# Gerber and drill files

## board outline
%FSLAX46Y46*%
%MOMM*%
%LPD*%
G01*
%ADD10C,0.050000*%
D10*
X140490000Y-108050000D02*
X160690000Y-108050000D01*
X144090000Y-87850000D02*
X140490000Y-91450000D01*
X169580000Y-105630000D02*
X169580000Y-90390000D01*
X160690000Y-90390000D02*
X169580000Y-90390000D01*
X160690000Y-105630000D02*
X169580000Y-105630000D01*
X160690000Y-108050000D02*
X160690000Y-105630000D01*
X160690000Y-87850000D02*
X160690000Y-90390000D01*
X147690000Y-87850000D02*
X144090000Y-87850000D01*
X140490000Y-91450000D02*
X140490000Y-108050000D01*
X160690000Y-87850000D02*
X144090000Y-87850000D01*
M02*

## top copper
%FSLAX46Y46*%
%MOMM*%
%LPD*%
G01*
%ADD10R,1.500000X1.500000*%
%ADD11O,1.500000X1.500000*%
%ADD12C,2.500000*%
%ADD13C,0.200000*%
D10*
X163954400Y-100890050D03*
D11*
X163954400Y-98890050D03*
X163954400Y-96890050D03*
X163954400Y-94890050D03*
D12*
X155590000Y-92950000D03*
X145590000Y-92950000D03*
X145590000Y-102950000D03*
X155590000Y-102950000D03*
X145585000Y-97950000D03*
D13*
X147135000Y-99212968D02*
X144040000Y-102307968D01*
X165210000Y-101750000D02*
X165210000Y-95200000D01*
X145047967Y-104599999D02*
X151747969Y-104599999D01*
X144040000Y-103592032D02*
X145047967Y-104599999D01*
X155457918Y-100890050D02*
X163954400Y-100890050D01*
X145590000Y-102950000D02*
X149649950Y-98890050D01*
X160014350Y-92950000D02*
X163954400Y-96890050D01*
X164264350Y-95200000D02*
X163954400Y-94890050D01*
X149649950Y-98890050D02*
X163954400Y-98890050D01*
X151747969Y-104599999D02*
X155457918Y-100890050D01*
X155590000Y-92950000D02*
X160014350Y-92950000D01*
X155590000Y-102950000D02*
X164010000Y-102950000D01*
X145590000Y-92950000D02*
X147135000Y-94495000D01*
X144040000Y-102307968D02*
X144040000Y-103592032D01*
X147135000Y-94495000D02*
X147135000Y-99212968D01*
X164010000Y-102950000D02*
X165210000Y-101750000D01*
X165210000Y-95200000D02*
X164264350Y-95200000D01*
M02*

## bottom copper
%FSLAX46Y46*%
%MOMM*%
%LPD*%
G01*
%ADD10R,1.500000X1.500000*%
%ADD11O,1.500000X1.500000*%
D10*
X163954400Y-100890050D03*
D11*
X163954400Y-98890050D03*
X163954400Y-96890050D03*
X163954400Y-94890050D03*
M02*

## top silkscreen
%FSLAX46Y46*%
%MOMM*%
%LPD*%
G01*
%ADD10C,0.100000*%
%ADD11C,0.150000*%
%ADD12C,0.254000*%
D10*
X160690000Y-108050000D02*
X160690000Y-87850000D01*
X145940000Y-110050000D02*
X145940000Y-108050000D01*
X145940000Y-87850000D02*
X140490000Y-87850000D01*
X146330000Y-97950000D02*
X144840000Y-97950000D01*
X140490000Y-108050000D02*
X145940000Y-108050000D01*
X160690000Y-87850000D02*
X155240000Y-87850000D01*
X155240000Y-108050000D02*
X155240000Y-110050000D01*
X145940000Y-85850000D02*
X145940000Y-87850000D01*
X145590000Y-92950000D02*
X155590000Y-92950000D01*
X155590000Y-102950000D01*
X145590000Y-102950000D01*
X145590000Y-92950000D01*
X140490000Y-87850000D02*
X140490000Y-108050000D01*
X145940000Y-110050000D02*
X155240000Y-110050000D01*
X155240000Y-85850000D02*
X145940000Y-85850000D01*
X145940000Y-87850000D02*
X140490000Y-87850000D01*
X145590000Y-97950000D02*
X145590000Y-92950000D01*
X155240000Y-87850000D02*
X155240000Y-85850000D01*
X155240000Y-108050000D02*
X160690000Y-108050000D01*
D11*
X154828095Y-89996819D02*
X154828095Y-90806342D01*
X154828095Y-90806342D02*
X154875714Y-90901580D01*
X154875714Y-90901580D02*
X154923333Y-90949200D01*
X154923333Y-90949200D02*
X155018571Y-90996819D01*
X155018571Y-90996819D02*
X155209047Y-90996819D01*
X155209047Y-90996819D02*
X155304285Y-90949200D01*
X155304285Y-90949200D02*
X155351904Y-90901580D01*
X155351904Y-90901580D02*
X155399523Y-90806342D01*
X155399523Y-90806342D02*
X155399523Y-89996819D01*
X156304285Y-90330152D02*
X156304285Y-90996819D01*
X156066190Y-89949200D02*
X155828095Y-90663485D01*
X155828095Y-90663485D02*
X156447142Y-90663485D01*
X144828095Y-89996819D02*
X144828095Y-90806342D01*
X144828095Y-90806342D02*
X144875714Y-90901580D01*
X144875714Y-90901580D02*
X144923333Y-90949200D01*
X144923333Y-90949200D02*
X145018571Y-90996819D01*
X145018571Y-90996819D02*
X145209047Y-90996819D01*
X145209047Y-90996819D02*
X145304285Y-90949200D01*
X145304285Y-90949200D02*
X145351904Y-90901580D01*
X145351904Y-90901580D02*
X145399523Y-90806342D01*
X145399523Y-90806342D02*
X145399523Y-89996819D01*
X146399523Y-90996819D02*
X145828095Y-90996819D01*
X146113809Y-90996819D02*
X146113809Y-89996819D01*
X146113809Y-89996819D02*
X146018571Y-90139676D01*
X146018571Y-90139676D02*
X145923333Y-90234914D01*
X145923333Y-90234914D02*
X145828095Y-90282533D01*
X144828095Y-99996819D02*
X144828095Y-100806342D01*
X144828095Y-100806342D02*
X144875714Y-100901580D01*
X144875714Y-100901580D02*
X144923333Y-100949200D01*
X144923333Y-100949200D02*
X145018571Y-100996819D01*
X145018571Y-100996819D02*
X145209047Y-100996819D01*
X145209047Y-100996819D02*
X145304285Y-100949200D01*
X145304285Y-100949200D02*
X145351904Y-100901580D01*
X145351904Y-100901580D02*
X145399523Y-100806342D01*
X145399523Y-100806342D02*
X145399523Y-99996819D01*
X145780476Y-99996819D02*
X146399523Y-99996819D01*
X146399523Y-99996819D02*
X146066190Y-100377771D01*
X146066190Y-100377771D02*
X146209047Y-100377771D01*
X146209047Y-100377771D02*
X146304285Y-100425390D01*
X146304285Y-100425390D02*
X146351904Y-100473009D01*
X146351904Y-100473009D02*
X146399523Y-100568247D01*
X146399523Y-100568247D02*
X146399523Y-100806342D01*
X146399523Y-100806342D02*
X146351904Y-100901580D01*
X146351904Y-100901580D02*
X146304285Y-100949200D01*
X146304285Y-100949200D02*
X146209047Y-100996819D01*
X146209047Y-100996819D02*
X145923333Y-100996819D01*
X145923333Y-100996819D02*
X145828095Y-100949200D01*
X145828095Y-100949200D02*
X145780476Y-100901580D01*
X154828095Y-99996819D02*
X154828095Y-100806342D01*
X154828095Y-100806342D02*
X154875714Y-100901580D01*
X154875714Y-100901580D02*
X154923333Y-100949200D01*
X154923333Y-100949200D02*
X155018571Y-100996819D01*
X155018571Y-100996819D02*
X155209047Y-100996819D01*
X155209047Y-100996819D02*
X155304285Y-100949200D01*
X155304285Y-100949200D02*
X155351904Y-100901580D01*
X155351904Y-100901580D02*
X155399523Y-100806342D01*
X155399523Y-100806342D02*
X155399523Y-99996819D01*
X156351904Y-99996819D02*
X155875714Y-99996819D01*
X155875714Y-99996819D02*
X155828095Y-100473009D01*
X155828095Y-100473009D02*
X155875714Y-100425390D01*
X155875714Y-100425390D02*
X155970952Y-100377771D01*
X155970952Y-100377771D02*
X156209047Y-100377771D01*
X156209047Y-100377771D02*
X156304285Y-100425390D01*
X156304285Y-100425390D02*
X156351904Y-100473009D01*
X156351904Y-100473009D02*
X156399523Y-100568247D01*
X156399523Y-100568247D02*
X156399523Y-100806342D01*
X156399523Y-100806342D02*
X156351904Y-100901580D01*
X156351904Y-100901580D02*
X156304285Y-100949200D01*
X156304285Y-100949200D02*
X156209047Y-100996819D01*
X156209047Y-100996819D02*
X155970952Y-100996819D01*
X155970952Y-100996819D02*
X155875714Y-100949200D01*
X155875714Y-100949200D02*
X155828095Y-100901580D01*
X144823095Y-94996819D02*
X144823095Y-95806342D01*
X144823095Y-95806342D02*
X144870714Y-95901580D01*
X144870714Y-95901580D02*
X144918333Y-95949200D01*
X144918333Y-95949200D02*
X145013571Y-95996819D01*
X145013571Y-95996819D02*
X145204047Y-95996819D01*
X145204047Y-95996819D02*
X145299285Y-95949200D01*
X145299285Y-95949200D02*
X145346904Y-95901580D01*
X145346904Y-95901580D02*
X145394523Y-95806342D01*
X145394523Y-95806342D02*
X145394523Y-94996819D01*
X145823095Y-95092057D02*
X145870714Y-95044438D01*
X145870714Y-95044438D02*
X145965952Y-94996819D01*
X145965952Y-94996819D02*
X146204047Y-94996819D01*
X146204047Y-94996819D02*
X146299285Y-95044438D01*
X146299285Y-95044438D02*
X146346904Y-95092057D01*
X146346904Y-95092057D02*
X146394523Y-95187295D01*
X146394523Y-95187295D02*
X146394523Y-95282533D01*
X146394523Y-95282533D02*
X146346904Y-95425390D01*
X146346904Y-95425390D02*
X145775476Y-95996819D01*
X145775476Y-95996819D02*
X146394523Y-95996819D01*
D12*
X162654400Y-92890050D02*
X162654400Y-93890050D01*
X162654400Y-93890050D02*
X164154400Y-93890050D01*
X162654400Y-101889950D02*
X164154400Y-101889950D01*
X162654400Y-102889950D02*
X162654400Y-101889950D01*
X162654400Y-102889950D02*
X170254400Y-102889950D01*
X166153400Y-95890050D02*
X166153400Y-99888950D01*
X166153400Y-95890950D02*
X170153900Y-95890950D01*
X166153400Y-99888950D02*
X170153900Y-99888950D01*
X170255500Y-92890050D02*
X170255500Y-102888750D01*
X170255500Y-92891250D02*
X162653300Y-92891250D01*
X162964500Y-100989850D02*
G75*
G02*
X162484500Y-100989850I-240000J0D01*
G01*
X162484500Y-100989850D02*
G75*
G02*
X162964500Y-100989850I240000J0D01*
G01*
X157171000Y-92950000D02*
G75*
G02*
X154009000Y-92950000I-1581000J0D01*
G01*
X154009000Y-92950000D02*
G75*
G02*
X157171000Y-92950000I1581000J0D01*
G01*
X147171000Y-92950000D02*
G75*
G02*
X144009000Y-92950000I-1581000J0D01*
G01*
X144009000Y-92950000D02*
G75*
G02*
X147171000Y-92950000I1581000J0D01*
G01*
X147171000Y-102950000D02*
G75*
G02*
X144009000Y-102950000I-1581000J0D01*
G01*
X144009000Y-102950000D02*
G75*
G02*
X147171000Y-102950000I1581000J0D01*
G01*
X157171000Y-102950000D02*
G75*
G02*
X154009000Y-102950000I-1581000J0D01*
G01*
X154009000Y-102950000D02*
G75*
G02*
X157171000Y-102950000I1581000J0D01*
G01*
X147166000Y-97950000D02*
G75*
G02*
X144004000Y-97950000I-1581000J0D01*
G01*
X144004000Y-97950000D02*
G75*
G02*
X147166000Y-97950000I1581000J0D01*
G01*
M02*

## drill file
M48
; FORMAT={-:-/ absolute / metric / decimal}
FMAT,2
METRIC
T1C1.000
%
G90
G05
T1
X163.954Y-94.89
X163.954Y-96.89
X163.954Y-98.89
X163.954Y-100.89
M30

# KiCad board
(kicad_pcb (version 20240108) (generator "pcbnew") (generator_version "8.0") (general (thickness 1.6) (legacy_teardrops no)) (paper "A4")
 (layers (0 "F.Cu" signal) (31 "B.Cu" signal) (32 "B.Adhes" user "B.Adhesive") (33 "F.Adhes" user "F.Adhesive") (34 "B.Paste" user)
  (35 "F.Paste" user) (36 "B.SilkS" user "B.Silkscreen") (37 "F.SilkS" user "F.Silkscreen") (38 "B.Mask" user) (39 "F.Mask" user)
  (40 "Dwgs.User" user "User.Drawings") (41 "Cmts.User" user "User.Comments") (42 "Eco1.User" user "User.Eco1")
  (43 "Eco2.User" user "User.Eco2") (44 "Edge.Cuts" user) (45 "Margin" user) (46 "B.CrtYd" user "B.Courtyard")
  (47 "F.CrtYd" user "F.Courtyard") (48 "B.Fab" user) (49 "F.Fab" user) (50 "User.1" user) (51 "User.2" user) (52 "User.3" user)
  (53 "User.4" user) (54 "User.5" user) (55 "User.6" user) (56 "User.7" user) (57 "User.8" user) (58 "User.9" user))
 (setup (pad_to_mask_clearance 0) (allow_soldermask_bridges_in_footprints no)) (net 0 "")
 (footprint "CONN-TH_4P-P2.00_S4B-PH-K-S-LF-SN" (layer "F.Cu") (at 163.9544 97.89005 90)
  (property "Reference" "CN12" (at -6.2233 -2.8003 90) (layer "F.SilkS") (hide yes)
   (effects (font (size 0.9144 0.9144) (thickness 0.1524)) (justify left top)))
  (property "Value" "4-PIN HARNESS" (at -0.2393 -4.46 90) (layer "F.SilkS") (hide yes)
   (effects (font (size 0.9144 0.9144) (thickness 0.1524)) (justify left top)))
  (fp_line (start 5 -1.3) (end 4 -1.3) (stroke (width 0.254) (type default)) (layer "F.SilkS"))
  (fp_line (start 4 -1.3) (end 4 0.2) (stroke (width 0.254) (type default)) (layer "F.SilkS"))
  (fp_line (start -3.9999 -1.3) (end -3.9999 0.2) (stroke (width 0.254) (type default)) (layer "F.SilkS"))
  (fp_line (start -4.9999 -1.3) (end -3.9999 -1.3) (stroke (width 0.254) (type default)) (layer "F.SilkS"))
  (fp_line (start -4.9999 -1.3) (end -4.9999 6.3) (stroke (width 0.254) (type default)) (layer "F.SilkS"))
  (fp_line (start 2 2.199) (end -1.9989 2.199) (stroke (width 0.254) (type default)) (layer "F.SilkS"))
  (fp_line (start 1.9991 2.199) (end 1.9991 6.1995) (stroke (width 0.254) (type default)) (layer "F.SilkS"))
  (fp_line (start -1.9989 2.199) (end -1.9989 6.1995) (stroke (width 0.254) (type default)) (layer "F.SilkS"))
  (fp_line (start 5 6.3011) (end -4.9987 6.3011) (stroke (width 0.254) (type default)) (layer "F.SilkS"))
  (fp_line (start 4.9988 6.3011) (end 4.9988 -1.3011) (stroke (width 0.254) (type default)) (layer "F.SilkS"))
  (fp_circle (center -3.0998 -1.2299) (end -2.8598 -1.2299) (stroke (width 0.254) (type default)) (fill none) (layer "F.SilkS"))
  (pad "1" thru_hole rect (at -3 0 90) (size 1.5 1.5) (drill 1) (layers "*.Cu" "*.Mask") (remove_unused_layers no)
   (solder_mask_margin 0.0508) (thermal_bridge_angle 0))
  (pad "2" thru_hole oval (at -1 0 90) (size 1.5 1.5) (drill 1) (layers "*.Cu" "*.Mask") (remove_unused_layers no)
   (solder_mask_margin 0.0508) (thermal_bridge_angle 0))
  (pad "3" thru_hole oval (at 1 0 90) (size 1.5 1.5) (drill 1) (layers "*.Cu" "*.Mask") (remove_unused_layers no)
   (solder_mask_margin 0.0508) (thermal_bridge_angle 0))
  (pad "4" thru_hole oval (at 3 0 90) (size 1.5 1.5) (drill 1) (layers "*.Cu" "*.Mask") (remove_unused_layers no)
   (solder_mask_margin 0.0508) (thermal_bridge_angle 0))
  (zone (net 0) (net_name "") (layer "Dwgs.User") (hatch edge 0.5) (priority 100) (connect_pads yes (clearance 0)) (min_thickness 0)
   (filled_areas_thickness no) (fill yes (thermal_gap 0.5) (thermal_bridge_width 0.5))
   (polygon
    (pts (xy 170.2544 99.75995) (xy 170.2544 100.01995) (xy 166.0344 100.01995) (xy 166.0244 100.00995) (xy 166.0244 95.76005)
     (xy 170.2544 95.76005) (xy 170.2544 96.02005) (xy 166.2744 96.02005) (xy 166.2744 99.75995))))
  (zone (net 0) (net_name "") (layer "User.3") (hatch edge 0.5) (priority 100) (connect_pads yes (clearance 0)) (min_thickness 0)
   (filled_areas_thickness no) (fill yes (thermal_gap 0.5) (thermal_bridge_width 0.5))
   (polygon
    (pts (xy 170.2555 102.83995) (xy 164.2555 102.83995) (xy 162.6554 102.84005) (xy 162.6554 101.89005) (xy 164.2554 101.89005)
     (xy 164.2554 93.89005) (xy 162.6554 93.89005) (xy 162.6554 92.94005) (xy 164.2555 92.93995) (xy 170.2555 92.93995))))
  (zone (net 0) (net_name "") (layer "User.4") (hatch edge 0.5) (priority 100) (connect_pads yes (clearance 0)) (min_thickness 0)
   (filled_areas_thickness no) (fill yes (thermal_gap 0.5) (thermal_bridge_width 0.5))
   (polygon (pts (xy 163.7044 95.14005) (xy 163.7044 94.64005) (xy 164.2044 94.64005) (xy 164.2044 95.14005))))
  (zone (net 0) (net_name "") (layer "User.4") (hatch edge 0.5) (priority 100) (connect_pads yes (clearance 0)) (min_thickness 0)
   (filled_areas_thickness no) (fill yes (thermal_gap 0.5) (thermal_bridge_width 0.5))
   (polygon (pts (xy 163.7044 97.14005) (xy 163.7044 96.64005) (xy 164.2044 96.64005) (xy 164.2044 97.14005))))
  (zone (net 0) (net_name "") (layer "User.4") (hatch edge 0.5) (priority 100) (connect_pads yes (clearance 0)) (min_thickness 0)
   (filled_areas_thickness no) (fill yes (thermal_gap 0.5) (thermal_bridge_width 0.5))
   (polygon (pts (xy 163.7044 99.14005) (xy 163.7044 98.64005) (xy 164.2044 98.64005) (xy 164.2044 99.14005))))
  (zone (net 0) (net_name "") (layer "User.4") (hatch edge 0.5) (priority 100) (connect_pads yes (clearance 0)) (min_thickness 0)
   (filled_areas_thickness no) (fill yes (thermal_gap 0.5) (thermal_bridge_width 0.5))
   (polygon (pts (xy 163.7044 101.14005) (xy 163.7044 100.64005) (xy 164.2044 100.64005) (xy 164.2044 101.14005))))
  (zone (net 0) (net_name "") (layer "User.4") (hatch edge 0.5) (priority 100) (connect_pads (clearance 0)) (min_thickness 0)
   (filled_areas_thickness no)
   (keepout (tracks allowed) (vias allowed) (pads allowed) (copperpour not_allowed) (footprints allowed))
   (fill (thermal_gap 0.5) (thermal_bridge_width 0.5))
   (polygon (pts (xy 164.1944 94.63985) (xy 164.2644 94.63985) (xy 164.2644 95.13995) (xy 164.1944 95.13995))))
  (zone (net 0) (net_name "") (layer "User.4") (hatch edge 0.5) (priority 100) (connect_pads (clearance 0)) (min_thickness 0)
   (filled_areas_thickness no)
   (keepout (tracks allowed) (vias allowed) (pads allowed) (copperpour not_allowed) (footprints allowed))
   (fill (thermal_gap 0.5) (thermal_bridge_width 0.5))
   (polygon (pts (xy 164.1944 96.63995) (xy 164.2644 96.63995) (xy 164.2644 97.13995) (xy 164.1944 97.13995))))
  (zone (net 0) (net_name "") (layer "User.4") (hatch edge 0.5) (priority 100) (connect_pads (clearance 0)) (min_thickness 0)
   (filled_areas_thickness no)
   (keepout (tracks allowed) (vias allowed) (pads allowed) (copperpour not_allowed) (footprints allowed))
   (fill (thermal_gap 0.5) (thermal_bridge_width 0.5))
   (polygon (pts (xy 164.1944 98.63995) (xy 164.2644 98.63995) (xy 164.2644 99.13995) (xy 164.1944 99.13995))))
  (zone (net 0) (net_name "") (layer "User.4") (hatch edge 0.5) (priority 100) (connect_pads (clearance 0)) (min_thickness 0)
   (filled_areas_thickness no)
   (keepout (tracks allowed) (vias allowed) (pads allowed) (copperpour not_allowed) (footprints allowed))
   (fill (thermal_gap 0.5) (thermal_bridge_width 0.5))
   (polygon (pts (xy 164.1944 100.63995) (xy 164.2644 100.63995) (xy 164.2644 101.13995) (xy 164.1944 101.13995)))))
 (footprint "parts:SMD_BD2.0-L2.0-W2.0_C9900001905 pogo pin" (layer "F.Cu") (at 155.59 92.95)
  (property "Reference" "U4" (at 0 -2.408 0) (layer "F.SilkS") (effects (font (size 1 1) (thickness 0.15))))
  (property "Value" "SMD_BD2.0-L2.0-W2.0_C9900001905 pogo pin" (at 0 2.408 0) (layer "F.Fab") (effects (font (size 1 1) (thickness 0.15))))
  (fp_circle (center 0 0) (end 1.581 0) (stroke (width 0.254) (type default)) (fill none) (layer "F.SilkS"))
  (pad "1" smd circle (at 0 0) (size 2.5 2.5) (layers "F.Cu" "F.Paste" "F.Mask") (thermal_bridge_angle 90)))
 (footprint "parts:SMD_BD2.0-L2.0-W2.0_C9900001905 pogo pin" (layer "F.Cu") (at 145.59 92.95)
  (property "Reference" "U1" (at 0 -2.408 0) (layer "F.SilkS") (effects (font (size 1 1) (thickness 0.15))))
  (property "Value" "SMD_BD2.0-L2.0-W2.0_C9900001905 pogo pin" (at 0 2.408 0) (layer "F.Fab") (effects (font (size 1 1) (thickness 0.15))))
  (fp_circle (center 0 0) (end 1.581 0) (stroke (width 0.254) (type default)) (fill none) (layer "F.SilkS"))
  (pad "1" smd circle (at 0 0) (size 2.5 2.5) (layers "F.Cu" "F.Paste" "F.Mask") (thermal_bridge_angle 90)))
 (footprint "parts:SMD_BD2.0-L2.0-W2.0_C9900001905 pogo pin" (layer "F.Cu") (at 145.59 102.95)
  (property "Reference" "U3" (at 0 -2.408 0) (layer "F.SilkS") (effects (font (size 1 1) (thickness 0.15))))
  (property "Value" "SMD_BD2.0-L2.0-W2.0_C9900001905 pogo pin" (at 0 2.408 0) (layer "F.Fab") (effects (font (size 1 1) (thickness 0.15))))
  (fp_circle (center 0 0) (end 1.581 0) (stroke (width 0.254) (type default)) (fill none) (layer "F.SilkS"))
  (pad "1" smd circle (at 0 0) (size 2.5 2.5) (layers "F.Cu" "F.Paste" "F.Mask") (thermal_bridge_angle 90)))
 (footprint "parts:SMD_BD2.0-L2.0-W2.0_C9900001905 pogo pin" (layer "F.Cu") (at 155.59 102.95)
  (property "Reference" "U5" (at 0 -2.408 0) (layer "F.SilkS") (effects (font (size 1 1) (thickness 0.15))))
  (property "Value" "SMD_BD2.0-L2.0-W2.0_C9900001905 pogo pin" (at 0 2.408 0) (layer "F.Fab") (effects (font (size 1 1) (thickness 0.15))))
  (fp_circle (center 0 0) (end 1.581 0) (stroke (width 0.254) (type default)) (fill none) (layer "F.SilkS"))
  (pad "1" smd circle (at 0 0) (size 2.5 2.5) (layers "F.Cu" "F.Paste" "F.Mask") (thermal_bridge_angle 90)))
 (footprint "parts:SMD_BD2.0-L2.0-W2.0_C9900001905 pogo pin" (layer "F.Cu") (at 145.585 97.95)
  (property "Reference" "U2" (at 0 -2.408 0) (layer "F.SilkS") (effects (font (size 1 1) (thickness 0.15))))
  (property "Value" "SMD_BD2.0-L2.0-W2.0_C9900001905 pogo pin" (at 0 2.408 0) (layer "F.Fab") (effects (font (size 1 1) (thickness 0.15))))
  (fp_circle (center 0 0) (end 1.581 0) (stroke (width 0.254) (type default)) (fill none) (layer "F.SilkS"))
  (pad "1" smd circle (at 0 0) (size 2.5 2.5) (layers "F.Cu" "F.Paste" "F.Mask") (thermal_bridge_angle 90)))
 (gr_line (start 160.69 108.05) (end 160.69 87.85) (stroke (width 0.1) (type default)) (layer "F.SilkS"))
 (gr_line (start 145.94 110.05) (end 145.94 108.05) (stroke (width 0.1) (type default)) (layer "F.SilkS"))
 (gr_line (start 145.94 87.85) (end 140.49 87.85) (stroke (width 0.1) (type default)) (layer "F.SilkS"))
 (gr_line (start 146.33 97.95) (end 144.84 97.95) (stroke (width 0.1) (type default)) (layer "F.SilkS"))
 (gr_line (start 140.49 108.05) (end 145.94 108.05) (stroke (width 0.1) (type default)) (layer "F.SilkS"))
 (gr_line (start 160.69 87.85) (end 155.24 87.85) (stroke (width 0.1) (type default)) (layer "F.SilkS"))
 (gr_line (start 155.24 108.05) (end 155.24 110.05) (stroke (width 0.1) (type default)) (layer "F.SilkS"))
 (gr_line (start 145.94 85.85) (end 145.94 87.85) (stroke (width 0.1) (type default)) (layer "F.SilkS"))
 (gr_rect (start 145.59 92.95) (end 155.59 102.95) (stroke (width 0.1) (type default)) (fill none) (layer "F.SilkS"))
 (gr_line (start 140.49 87.85) (end 140.49 108.05) (stroke (width 0.1) (type default)) (layer "F.SilkS"))
 (gr_line (start 145.94 110.05) (end 155.24 110.05) (stroke (width 0.1) (type default)) (layer "F.SilkS"))
 (gr_line (start 155.24 85.85) (end 145.94 85.85) (stroke (width 0.1) (type default)) (layer "F.SilkS"))
 (gr_line (start 145.94 87.85) (end 140.49 87.85) (stroke (width 0.1) (type default)) (layer "F.SilkS"))
 (gr_line (start 145.59 97.95) (end 145.59 92.95) (stroke (width 0.1) (type default)) (layer "F.SilkS"))
 (gr_line (start 155.24 87.85) (end 155.24 85.85) (stroke (width 0.1) (type default)) (layer "F.SilkS"))
 (gr_line (start 155.24 108.05) (end 160.69 108.05) (stroke (width 0.1) (type default)) (layer "F.SilkS"))
 (gr_line (start 140.49 108.05) (end 160.69 108.05) (stroke (width 0.05) (type default)) (layer "Edge.Cuts"))
 (gr_line (start 144.09 87.85) (end 140.49 91.45) (stroke (width 0.05) (type default)) (layer "Edge.Cuts"))
 (gr_line (start 169.58 105.63) (end 169.58 90.39) (stroke (width 0.05) (type default)) (layer "Edge.Cuts"))
 (gr_line (start 160.69 90.39) (end 169.58 90.39) (stroke (width 0.05) (type default)) (layer "Edge.Cuts"))
 (gr_line (start 160.69 105.63) (end 169.58 105.63) (stroke (width 0.05) (type default)) (layer "Edge.Cuts"))
 (gr_line (start 160.69 108.05) (end 160.69 105.63) (stroke (width 0.05) (type default)) (layer "Edge.Cuts"))
 (gr_line (start 160.69 87.85) (end 160.69 90.39) (stroke (width 0.05) (type default)) (layer "Edge.Cuts"))
 (gr_line (start 147.69 87.85) (end 144.09 87.85) (stroke (width 0.05) (type default)) (layer "Edge.Cuts"))
 (gr_line (start 140.49 91.45) (end 140.49 108.05) (stroke (width 0.05) (type default)) (layer "Edge.Cuts"))
 (gr_line (start 160.69 87.85) (end 144.09 87.85) (stroke (width 0.05) (type default)) (layer "Edge.Cuts"))
 (segment (start 147.135 99.212968) (end 144.04 102.307968) (width 0.2) (layer "F.Cu") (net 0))
 (segment (start 165.21 101.75) (end 165.21 95.2) (width 0.2) (layer "F.Cu") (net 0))
 (segment (start 145.047967 104.599999) (end 151.747969 104.599999) (width 0.2) (layer "F.Cu") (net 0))
 (segment (start 144.04 103.592032) (end 145.047967 104.599999) (width 0.2) (layer "F.Cu") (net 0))
 (segment (start 155.457918 100.89005) (end 163.9544 100.89005) (width 0.2) (layer "F.Cu") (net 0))
 (segment (start 145.59 102.95) (end 149.64995 98.89005) (width 0.2) (layer "F.Cu") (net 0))
 (segment (start 160.01435 92.95) (end 163.9544 96.89005) (width 0.2) (layer "F.Cu") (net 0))
 (segment (start 164.26435 95.2) (end 163.9544 94.89005) (width 0.2) (layer "F.Cu") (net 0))
 (segment (start 149.64995 98.89005) (end 163.9544 98.89005) (width 0.2) (layer "F.Cu") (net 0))
 (segment (start 151.747969 104.599999) (end 155.457918 100.89005) (width 0.2) (layer "F.Cu") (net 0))
 (segment (start 155.59 92.95) (end 160.01435 92.95) (width 0.2) (layer "F.Cu") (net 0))
 (segment (start 155.59 102.95) (end 164.01 102.95) (width 0.2) (layer "F.Cu") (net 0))
 (segment (start 145.59 92.95) (end 147.135 94.495) (width 0.2) (layer "F.Cu") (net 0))
 (segment (start 144.04 102.307968) (end 144.04 103.592032) (width 0.2) (layer "F.Cu") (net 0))
 (segment (start 147.135 94.495) (end 147.135 99.212968) (width 0.2) (layer "F.Cu") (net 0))
 (segment (start 164.01 102.95) (end 165.21 101.75) (width 0.2) (layer "F.Cu") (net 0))
 (segment (start 165.21 95.2) (end 164.26435 95.2) (width 0.2) (layer "F.Cu") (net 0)))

